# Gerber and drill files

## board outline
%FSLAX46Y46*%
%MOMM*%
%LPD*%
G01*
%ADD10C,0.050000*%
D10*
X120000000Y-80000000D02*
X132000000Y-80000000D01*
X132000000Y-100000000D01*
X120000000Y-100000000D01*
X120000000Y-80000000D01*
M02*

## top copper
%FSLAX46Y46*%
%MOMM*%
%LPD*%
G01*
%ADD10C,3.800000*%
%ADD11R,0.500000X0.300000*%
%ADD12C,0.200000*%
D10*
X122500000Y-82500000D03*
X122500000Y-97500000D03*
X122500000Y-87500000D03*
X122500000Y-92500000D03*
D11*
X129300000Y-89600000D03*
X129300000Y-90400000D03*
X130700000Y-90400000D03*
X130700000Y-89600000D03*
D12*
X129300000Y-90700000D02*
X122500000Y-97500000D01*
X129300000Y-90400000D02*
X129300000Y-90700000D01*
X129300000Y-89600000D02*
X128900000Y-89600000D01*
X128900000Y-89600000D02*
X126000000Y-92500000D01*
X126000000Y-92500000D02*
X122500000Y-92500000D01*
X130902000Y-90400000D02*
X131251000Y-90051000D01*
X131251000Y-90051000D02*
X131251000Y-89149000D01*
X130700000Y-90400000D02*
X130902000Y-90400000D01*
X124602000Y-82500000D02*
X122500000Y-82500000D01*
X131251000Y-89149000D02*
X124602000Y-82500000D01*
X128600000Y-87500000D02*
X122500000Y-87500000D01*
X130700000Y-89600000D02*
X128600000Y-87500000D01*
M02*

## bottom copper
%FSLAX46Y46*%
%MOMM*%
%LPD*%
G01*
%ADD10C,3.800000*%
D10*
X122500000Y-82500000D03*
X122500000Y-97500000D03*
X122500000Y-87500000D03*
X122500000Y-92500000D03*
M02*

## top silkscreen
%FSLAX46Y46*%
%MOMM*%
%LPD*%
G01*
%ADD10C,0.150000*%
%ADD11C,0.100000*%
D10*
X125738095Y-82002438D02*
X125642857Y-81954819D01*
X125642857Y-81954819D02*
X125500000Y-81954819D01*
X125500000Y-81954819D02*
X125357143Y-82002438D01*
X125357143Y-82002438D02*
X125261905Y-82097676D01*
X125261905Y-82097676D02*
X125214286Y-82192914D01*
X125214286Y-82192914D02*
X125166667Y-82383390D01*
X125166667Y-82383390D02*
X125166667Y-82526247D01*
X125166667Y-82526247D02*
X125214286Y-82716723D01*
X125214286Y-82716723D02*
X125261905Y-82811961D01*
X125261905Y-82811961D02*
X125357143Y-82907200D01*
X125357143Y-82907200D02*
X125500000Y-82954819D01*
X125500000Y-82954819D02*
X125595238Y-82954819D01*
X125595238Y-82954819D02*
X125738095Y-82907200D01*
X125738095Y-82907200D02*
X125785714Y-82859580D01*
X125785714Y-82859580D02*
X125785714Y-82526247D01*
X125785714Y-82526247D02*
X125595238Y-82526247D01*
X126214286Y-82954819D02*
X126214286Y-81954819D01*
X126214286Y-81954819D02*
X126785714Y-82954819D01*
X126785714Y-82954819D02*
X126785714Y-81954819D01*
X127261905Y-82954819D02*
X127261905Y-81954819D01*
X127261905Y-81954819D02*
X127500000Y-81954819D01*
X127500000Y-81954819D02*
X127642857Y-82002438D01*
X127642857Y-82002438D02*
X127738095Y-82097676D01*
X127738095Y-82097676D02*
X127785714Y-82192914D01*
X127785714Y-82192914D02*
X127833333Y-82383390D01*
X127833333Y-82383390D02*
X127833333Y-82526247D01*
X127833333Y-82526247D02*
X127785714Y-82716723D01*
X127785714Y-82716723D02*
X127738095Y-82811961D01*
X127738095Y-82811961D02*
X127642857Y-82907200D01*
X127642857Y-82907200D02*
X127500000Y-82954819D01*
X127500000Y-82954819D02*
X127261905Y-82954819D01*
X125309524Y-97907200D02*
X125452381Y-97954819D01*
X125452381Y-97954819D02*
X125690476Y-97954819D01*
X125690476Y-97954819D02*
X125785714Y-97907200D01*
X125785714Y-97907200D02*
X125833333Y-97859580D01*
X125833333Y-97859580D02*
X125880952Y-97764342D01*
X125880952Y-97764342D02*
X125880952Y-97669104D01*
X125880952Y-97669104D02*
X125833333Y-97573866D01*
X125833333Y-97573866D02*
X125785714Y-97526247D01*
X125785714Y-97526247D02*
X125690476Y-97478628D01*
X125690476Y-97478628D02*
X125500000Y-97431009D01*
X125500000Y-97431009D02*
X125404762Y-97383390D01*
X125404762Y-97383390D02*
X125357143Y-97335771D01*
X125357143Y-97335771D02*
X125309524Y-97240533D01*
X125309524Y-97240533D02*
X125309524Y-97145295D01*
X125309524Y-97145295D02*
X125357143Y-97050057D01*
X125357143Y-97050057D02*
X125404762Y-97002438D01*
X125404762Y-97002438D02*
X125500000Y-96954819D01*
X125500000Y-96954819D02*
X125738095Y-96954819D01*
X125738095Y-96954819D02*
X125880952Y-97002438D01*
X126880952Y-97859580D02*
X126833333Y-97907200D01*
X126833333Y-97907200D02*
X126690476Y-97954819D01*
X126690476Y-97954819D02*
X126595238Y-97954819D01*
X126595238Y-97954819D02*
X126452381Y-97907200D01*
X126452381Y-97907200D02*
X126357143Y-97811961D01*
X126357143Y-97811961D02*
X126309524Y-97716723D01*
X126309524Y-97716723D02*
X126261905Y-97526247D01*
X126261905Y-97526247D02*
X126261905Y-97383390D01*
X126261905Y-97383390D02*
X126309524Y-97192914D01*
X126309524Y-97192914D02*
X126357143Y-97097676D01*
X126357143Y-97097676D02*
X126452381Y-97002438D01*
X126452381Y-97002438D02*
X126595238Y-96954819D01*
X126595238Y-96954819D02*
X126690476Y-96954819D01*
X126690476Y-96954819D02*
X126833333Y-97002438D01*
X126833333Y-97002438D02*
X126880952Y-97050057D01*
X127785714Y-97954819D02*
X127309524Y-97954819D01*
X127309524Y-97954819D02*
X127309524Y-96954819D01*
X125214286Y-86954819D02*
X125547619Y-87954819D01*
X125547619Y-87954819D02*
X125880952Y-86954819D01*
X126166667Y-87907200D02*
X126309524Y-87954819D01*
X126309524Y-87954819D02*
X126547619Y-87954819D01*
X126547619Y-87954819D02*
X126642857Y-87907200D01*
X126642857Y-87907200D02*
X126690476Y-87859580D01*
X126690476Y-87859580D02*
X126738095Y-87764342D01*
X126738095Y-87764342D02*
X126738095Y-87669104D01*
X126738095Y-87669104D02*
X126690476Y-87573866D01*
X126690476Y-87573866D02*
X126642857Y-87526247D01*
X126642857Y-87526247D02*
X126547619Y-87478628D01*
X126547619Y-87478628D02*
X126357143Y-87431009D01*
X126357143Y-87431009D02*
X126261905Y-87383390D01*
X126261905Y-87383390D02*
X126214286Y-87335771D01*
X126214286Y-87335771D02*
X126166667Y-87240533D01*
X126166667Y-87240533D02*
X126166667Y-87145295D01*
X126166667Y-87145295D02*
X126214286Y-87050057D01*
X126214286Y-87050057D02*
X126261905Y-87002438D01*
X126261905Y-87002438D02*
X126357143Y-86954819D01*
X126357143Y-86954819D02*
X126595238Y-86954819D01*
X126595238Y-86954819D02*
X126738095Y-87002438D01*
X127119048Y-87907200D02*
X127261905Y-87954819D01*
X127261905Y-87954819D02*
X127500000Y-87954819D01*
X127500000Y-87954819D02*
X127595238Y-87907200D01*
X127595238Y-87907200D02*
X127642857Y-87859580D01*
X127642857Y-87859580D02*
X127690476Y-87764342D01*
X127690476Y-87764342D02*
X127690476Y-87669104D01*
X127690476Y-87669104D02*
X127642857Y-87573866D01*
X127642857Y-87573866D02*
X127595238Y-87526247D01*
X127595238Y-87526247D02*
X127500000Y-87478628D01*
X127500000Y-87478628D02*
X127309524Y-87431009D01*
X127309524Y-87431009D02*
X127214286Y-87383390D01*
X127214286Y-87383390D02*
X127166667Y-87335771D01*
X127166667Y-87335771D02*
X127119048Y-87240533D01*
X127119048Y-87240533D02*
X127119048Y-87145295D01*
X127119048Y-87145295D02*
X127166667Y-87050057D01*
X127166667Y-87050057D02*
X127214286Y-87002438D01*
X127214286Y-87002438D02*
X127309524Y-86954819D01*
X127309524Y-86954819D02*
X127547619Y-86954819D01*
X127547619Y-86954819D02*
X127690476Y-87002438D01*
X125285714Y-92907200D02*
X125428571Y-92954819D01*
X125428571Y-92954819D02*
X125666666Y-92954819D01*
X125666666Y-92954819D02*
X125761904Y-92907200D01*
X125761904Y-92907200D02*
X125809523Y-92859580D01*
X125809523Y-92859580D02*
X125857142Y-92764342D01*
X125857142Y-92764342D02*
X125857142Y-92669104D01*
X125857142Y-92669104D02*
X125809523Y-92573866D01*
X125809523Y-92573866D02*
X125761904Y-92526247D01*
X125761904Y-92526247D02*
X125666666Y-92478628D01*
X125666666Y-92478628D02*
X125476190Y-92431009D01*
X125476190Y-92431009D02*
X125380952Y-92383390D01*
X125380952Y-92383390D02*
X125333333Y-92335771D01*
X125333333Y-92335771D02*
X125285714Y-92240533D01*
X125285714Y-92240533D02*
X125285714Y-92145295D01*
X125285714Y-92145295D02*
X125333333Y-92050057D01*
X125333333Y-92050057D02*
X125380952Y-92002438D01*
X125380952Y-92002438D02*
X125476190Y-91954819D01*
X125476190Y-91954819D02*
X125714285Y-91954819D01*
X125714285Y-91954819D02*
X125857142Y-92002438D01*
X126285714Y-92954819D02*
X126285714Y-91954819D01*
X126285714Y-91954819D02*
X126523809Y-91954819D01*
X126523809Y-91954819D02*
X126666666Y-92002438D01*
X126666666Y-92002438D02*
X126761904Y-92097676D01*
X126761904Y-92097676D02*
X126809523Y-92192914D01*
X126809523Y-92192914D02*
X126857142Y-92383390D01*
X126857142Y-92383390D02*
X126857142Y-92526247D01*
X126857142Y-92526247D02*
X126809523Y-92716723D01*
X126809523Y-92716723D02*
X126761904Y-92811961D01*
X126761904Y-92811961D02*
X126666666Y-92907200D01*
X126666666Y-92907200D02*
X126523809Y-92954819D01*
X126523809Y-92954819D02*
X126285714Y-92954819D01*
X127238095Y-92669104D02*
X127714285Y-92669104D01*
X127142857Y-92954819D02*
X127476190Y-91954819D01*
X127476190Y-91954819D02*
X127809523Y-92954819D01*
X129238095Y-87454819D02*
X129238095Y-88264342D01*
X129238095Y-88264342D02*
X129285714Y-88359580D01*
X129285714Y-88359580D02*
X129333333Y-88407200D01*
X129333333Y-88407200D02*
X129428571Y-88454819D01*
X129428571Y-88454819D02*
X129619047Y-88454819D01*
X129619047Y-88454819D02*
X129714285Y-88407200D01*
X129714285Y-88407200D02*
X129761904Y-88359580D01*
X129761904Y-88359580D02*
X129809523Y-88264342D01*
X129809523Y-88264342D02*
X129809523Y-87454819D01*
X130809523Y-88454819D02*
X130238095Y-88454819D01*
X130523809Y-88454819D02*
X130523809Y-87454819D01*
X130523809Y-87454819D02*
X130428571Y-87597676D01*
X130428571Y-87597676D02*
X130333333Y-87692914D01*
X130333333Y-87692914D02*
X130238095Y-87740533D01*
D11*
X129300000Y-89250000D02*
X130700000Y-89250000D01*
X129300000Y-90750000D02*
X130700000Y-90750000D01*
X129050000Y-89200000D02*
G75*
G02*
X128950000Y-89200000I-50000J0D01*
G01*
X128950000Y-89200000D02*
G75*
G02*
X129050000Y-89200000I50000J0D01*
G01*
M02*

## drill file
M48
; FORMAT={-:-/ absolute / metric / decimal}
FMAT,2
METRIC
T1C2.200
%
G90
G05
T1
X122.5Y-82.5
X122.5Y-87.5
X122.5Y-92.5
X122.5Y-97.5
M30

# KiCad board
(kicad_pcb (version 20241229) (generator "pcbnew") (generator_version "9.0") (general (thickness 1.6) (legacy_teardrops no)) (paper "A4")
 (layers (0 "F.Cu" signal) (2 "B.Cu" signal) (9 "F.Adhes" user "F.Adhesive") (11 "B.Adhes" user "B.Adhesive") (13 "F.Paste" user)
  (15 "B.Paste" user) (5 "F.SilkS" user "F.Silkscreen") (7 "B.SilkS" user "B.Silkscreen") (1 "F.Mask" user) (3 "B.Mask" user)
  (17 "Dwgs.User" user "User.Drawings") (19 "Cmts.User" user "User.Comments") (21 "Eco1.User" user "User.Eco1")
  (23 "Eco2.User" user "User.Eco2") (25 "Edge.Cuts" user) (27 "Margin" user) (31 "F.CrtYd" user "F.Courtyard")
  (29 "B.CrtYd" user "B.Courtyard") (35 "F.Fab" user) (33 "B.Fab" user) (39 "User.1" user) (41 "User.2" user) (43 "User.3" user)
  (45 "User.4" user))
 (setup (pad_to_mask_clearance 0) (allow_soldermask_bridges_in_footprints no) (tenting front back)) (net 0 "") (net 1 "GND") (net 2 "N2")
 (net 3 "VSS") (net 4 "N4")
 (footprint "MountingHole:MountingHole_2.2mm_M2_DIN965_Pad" (layer "F.Cu") (at 122.5 82.5)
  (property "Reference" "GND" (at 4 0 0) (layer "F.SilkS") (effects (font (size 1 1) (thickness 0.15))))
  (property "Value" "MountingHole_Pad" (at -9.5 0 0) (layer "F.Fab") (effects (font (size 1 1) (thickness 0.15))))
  (pad "1" thru_hole circle (at 0 0) (size 3.8 3.8) (drill 2.2) (layers "*.Cu" "*.Mask") (remove_unused_layers no) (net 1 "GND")
   (zone_connect 2)))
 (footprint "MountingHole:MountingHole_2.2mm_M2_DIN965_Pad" (layer "F.Cu") (at 122.5 97.5)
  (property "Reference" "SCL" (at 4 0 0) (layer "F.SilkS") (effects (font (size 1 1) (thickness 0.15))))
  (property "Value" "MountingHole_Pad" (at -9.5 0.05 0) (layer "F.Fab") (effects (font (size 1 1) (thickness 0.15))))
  (pad "1" thru_hole circle (at 0 0) (size 3.8 3.8) (drill 2.2) (layers "*.Cu" "*.Mask") (remove_unused_layers no) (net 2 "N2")
   (zone_connect 2)))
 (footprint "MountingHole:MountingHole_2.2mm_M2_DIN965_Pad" (layer "F.Cu") (at 122.5 87.5)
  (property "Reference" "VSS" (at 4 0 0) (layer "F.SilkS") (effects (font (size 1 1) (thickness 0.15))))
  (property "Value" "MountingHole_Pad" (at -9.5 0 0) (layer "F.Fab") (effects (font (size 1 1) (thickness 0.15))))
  (pad "1" thru_hole circle (at 0 0) (size 3.8 3.8) (drill 2.2) (layers "*.Cu" "*.Mask") (remove_unused_layers no) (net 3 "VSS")
   (zone_connect 2)))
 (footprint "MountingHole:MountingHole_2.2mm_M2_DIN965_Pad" (layer "F.Cu") (at 122.5 92.5)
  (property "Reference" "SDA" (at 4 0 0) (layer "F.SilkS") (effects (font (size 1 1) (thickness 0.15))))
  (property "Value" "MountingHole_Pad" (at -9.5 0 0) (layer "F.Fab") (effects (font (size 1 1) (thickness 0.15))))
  (pad "1" thru_hole circle (at 0 0) (size 3.8 3.8) (drill 2.2) (layers "*.Cu" "*.Mask") (remove_unused_layers no) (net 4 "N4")
   (zone_connect 2)))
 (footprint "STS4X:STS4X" (layer "F.Cu") (at 130 90)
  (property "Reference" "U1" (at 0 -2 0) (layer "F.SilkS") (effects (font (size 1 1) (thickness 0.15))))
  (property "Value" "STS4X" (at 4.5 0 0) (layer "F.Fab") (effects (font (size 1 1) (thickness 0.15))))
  (fp_line (start -0.7 -0.75) (end 0.7 -0.75) (stroke (width 0.1) (type solid)) (layer "F.SilkS"))
  (fp_line (start -0.7 0.75) (end 0.7 0.75) (stroke (width 0.1) (type solid)) (layer "F.SilkS"))
  (fp_circle (center -1 -0.8) (end -0.95 -0.8) (stroke (width 0.1) (type solid)) (fill no) (layer "F.SilkS"))
  (pad "1" smd rect (at -0.7 -0.4) (size 0.5 0.3) (layers "F.Cu" "F.Mask" "F.Paste") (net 4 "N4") (solder_mask_margin 0.102))
  (pad "2" smd rect (at -0.7 0.4) (size 0.5 0.3) (layers "F.Cu" "F.Mask" "F.Paste") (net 2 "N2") (solder_mask_margin 0.102))
  (pad "3" smd rect (at 0.7 0.4) (size 0.5 0.3) (layers "F.Cu" "F.Mask" "F.Paste") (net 1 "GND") (solder_mask_margin 0.102))
  (pad "4" smd rect (at 0.7 -0.4) (size 0.5 0.3) (layers "F.Cu" "F.Mask" "F.Paste") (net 3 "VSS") (solder_mask_margin 0.102)))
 (gr_rect (start 120 80) (end 132 100) (stroke (width 0.05) (type default)) (fill no) (layer "Edge.Cuts"))
 (segment (start 129.3 90.7) (end 122.5 97.5) (width 0.2) (layer "F.Cu") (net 2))
 (segment (start 129.3 90.4) (end 129.3 90.7) (width 0.2) (layer "F.Cu") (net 2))
 (segment (start 129.3 89.6) (end 128.9 89.6) (width 0.2) (layer "F.Cu") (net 4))
 (segment (start 128.9 89.6) (end 126 92.5) (width 0.2) (layer "F.Cu") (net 4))
 (segment (start 126 92.5) (end 122.5 92.5) (width 0.2) (layer "F.Cu") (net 4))
 (segment (start 130.902 90.4) (end 131.251 90.051) (width 0.2) (layer "F.Cu") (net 1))
 (segment (start 131.251 90.051) (end 131.251 89.149) (width 0.2) (layer "F.Cu") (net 1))
 (segment (start 130.7 90.4) (end 130.902 90.4) (width 0.2) (layer "F.Cu") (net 1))
 (segment (start 124.602 82.5) (end 122.5 82.5) (width 0.2) (layer "F.Cu") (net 1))
 (segment (start 131.251 89.149) (end 124.602 82.5) (width 0.2) (layer "F.Cu") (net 1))
 (segment (start 128.6 87.5) (end 122.5 87.5) (width 0.2) (layer "F.Cu") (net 3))
 (segment (start 130.7 89.6) (end 128.6 87.5) (width 0.2) (layer "F.Cu") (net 3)))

